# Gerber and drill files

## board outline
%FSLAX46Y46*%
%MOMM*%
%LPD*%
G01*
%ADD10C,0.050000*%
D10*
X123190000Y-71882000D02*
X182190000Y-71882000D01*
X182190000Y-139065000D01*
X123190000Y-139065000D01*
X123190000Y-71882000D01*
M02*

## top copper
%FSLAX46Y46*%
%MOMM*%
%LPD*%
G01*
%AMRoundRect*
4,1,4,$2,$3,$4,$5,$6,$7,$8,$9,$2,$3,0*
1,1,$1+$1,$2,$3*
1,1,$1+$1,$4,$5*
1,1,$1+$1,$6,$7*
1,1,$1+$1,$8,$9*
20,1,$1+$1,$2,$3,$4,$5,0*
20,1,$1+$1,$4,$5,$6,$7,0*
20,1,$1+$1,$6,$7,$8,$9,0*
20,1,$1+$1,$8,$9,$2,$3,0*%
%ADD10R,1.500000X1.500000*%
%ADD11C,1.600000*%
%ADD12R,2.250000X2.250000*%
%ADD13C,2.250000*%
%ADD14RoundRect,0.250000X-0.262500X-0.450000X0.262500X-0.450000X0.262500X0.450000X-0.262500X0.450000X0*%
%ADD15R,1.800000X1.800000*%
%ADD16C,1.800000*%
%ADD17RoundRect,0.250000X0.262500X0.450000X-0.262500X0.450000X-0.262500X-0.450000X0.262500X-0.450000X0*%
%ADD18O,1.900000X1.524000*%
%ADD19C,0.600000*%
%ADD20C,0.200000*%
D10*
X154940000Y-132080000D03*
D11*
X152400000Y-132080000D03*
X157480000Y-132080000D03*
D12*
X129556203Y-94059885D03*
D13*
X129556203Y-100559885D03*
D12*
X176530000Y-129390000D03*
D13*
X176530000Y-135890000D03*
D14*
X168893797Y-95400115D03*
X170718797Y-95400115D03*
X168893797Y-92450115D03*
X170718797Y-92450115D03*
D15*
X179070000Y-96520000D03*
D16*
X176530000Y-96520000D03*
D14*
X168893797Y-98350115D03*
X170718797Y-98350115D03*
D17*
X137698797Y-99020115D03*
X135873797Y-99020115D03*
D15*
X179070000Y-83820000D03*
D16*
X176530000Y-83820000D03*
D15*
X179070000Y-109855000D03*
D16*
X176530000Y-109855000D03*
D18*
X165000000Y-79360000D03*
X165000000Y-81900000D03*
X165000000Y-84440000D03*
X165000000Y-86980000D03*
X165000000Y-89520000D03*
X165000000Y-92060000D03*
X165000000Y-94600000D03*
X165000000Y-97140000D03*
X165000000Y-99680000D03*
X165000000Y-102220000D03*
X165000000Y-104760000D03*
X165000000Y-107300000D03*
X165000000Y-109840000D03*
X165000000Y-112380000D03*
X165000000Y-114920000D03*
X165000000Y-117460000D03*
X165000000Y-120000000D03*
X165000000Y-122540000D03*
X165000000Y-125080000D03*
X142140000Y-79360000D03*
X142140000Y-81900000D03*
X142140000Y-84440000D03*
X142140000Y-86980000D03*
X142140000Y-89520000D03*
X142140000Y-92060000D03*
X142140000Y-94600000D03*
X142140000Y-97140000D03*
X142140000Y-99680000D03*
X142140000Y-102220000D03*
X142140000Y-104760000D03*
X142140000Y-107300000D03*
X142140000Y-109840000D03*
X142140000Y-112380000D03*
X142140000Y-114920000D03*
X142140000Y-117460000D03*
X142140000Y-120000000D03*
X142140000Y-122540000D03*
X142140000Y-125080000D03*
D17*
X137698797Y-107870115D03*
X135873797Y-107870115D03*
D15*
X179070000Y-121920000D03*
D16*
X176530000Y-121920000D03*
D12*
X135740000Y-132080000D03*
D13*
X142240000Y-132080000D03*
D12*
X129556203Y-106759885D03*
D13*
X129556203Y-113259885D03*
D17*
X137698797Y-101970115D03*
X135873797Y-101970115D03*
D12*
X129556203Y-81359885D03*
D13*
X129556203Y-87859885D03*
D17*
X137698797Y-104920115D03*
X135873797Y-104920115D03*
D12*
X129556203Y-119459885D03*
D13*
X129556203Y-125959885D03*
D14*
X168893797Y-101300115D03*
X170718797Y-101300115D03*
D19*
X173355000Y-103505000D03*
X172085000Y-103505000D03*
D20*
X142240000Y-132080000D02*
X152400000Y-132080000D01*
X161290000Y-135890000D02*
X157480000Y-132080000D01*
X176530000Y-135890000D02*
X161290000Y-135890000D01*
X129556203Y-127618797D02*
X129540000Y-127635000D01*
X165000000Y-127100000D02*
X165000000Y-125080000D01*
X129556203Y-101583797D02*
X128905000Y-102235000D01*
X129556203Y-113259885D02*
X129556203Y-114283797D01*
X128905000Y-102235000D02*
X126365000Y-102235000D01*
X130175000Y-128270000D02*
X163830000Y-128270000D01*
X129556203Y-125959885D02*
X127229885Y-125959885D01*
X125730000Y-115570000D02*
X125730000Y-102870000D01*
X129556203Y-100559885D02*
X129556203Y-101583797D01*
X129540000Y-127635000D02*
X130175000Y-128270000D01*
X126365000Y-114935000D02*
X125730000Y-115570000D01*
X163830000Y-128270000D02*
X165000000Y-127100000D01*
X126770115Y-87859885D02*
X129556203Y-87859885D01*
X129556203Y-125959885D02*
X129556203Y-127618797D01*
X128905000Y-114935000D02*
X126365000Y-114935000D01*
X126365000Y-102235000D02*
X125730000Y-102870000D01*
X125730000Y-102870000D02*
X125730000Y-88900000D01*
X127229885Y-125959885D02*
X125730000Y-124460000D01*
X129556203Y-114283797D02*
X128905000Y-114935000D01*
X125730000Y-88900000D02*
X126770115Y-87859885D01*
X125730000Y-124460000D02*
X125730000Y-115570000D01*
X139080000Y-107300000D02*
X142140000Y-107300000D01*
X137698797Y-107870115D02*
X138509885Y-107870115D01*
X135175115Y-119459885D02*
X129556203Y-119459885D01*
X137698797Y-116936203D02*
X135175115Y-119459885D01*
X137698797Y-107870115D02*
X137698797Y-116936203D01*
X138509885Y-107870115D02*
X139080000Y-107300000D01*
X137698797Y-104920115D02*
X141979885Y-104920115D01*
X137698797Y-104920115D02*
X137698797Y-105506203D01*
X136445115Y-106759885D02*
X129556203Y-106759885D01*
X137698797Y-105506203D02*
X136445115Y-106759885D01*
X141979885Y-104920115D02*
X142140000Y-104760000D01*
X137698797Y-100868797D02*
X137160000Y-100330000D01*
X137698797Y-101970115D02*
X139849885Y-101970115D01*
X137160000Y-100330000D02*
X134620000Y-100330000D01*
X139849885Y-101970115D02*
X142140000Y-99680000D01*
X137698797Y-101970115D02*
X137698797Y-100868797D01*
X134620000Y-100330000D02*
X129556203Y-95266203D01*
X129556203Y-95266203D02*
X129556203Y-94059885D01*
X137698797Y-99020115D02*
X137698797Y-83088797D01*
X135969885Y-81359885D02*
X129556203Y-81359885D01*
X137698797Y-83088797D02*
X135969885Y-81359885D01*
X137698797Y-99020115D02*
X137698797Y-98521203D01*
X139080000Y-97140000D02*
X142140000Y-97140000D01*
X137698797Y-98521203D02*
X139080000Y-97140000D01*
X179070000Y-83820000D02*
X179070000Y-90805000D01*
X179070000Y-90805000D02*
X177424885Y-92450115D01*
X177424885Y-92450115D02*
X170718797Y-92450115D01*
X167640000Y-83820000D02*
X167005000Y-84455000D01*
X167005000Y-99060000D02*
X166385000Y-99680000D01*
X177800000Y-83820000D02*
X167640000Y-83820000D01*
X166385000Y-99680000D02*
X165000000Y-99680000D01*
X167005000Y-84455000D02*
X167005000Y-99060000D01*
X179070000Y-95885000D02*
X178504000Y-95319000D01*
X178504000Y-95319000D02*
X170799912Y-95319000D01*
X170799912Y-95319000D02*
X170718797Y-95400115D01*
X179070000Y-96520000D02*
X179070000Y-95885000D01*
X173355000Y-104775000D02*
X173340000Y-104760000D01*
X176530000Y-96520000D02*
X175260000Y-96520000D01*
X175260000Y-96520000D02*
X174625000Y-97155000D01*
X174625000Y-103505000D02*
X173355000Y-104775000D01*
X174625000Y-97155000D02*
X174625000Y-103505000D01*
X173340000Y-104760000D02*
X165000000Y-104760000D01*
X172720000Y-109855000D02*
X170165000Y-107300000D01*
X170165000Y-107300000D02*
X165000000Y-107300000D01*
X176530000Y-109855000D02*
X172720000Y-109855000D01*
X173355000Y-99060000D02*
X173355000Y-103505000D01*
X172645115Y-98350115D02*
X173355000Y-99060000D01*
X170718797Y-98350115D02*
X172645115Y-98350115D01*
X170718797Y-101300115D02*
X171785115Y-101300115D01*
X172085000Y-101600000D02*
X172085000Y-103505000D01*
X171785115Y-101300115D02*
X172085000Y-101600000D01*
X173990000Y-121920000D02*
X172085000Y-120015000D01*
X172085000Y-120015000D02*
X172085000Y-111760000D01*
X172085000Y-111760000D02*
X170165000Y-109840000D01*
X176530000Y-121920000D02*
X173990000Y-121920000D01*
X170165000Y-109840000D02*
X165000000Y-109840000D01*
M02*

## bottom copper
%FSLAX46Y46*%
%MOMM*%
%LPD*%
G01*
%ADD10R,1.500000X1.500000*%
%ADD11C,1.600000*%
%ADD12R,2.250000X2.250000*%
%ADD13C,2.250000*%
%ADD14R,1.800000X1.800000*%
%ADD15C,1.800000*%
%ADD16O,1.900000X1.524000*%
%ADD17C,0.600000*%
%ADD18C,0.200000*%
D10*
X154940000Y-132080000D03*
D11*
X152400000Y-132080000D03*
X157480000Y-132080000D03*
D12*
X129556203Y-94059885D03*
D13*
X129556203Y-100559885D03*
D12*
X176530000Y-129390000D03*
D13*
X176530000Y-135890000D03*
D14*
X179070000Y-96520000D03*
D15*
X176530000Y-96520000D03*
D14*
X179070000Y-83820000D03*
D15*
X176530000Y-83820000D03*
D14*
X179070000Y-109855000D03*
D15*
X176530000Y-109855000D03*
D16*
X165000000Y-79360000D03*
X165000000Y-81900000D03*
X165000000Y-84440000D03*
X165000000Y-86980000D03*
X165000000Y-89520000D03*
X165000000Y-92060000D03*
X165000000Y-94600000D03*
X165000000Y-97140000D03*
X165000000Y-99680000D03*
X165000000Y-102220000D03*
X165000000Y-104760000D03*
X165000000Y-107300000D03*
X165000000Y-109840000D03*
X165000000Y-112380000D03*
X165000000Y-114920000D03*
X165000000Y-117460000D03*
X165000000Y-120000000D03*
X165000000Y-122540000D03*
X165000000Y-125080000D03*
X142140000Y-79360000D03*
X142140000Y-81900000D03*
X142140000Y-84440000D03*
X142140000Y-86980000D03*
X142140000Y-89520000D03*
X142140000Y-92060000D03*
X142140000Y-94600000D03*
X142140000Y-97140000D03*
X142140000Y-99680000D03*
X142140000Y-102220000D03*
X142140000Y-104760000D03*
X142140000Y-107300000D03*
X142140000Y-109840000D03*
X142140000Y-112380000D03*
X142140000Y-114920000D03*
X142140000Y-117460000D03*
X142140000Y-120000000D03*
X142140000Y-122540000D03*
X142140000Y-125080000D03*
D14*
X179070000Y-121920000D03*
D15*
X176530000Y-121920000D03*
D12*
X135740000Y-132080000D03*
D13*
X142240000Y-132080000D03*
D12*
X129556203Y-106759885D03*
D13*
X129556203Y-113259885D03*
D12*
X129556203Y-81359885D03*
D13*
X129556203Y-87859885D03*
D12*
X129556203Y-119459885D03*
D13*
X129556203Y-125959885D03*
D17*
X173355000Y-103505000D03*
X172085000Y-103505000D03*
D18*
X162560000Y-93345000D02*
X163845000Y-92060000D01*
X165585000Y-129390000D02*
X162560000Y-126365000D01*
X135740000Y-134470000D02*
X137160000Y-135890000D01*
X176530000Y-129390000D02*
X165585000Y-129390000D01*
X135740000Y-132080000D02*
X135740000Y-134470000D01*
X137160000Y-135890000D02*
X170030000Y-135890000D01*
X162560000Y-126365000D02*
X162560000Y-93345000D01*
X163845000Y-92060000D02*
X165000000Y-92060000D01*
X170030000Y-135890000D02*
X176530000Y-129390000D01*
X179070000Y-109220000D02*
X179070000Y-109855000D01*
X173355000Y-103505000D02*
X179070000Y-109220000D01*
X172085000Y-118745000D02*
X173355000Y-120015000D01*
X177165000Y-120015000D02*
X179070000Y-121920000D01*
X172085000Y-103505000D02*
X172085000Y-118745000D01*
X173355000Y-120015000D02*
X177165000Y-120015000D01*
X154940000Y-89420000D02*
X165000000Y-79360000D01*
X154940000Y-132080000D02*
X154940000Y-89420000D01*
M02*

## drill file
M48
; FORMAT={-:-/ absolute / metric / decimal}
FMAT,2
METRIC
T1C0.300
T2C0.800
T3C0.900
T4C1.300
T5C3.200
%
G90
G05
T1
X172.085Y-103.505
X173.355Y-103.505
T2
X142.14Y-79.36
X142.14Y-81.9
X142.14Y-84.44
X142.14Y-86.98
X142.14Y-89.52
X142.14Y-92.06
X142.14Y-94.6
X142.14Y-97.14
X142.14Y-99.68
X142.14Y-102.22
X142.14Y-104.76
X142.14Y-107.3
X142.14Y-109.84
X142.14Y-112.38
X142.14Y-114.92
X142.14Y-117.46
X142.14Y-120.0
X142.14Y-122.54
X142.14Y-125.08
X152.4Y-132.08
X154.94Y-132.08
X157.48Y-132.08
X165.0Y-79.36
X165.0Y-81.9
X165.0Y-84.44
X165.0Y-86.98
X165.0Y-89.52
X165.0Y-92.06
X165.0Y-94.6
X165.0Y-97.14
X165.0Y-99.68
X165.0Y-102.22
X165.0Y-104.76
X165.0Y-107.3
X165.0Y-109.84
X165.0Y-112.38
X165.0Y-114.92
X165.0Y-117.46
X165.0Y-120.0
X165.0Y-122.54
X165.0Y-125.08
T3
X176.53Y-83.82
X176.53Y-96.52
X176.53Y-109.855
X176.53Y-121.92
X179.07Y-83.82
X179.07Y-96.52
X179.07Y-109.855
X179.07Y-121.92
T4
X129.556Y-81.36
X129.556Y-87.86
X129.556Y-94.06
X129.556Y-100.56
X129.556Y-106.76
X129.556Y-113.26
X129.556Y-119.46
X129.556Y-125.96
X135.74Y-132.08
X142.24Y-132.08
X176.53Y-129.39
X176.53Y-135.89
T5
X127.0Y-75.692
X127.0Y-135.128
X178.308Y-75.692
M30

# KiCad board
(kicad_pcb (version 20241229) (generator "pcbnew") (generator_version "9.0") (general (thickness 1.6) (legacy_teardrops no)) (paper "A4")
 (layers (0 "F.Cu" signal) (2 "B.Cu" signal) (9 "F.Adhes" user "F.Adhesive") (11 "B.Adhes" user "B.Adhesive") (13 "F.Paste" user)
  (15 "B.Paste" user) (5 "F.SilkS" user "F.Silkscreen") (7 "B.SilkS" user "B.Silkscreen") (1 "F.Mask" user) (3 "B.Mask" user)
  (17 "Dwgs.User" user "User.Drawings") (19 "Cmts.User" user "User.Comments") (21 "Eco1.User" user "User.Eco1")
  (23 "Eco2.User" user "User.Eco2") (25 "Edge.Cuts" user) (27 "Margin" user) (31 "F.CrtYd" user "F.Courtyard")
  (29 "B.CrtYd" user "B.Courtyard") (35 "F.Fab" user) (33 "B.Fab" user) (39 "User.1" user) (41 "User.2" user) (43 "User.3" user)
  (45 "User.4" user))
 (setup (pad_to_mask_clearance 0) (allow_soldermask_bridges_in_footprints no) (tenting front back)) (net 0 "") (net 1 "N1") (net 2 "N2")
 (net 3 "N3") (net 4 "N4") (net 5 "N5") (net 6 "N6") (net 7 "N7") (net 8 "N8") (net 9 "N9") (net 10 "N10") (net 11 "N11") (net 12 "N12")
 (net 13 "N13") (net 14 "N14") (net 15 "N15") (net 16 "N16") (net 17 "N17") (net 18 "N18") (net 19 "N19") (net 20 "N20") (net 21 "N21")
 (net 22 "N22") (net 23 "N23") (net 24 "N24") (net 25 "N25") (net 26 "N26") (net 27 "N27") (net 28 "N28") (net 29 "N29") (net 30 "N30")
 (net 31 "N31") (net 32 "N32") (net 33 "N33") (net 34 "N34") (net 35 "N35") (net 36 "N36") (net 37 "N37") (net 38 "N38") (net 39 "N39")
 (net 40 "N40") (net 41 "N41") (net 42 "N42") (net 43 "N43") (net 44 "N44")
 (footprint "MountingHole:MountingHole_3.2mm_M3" (layer "F.Cu") (at 178.308 75.692)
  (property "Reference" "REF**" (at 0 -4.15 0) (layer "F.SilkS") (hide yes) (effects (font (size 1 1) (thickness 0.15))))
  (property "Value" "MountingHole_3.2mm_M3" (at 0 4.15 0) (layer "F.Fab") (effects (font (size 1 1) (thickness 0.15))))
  (pad "" np_thru_hole circle (at 0 0) (size 3.2 3.2) (drill 3.2) (layers "*.Cu" "*.Mask")))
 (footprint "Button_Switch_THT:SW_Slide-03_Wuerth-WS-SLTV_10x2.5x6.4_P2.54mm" (layer "F.Cu") (at 154.94 132.08)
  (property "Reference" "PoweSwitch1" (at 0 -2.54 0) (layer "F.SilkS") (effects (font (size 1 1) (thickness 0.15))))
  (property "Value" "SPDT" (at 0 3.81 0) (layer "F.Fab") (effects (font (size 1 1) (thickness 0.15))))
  (pad "1" thru_hole rect (at 0 0) (size 1.5 1.5) (drill 0.8) (layers "*.Cu" "*.Mask") (remove_unused_layers no) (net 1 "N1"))
  (pad "2" thru_hole circle (at -2.54 0) (size 1.6 1.6) (drill 0.8) (layers "*.Cu" "*.Mask") (remove_unused_layers no) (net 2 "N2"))
  (pad "3" thru_hole circle (at 2.54 0) (size 1.6 1.6) (drill 0.8) (layers "*.Cu" "*.Mask") (remove_unused_layers no) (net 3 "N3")))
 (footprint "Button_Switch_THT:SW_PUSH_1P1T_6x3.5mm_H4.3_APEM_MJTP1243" (layer "F.Cu") (at 129.556203 94.059885 -90)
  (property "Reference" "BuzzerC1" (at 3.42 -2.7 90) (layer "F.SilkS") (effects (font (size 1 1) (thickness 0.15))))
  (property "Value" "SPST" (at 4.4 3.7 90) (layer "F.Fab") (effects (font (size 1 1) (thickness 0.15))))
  (pad "1" thru_hole rect (at 0 0) (size 2.25 2.25) (drill 1.3) (layers "*.Cu" "*.Mask") (remove_unused_layers no) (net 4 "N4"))
  (pad "2" thru_hole circle (at 6.5 0) (size 2.25 2.25) (drill 1.3) (layers "*.Cu" "*.Mask") (remove_unused_layers no) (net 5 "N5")))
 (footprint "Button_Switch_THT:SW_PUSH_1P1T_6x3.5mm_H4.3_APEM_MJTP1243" (layer "F.Cu") (at 176.53 129.39 -90)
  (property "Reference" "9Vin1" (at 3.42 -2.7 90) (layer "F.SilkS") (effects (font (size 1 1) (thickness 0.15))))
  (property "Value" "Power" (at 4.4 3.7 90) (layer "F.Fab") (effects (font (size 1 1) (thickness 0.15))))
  (pad "1" thru_hole rect (at 0 0) (size 2.25 2.25) (drill 1.3) (layers "*.Cu" "*.Mask") (remove_unused_layers no) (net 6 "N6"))
  (pad "2" thru_hole circle (at 6.5 0) (size 2.25 2.25) (drill 1.3) (layers "*.Cu" "*.Mask") (remove_unused_layers no) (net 3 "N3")))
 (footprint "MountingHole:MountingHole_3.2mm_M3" (layer "F.Cu") (at 127 135.128)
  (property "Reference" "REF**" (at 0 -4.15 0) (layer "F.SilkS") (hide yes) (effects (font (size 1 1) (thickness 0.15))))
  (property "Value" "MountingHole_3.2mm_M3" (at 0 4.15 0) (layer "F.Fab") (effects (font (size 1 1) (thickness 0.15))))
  (pad "" np_thru_hole circle (at 0 0) (size 3.2 3.2) (drill 3.2) (layers "*.Cu" "*.Mask")))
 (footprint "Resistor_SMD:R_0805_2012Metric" (layer "F.Cu") (at 169.806297 95.400115)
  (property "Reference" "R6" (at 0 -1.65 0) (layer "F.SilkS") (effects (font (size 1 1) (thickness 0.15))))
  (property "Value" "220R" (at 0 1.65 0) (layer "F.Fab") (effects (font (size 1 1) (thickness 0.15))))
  (pad "1" smd roundrect (at -0.9125 0) (size 1.025 1.4) (layers "F.Cu" "F.Mask" "F.Paste") (roundrect_rratio 0.243902) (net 6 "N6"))
  (pad "2" smd roundrect (at 0.9125 0) (size 1.025 1.4) (layers "F.Cu" "F.Mask" "F.Paste") (roundrect_rratio 0.243902) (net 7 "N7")))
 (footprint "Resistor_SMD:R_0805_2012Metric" (layer "F.Cu") (at 169.806297 92.450115)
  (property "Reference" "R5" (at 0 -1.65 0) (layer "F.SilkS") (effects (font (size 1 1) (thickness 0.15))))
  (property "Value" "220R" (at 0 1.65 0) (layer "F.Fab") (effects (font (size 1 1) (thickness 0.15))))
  (pad "1" smd roundrect (at -0.9125 0) (size 1.025 1.4) (layers "F.Cu" "F.Mask" "F.Paste") (roundrect_rratio 0.243902) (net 6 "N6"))
  (pad "2" smd roundrect (at 0.9125 0) (size 1.025 1.4) (layers "F.Cu" "F.Mask" "F.Paste") (roundrect_rratio 0.243902) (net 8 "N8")))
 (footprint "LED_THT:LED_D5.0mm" (layer "F.Cu") (at 179.07 96.52 180)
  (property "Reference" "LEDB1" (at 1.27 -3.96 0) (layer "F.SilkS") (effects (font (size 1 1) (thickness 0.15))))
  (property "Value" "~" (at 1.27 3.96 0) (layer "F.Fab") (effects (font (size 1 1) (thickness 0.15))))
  (pad "1" thru_hole rect (at 0 0 180) (size 1.8 1.8) (drill 0.9) (layers "*.Cu" "*.Mask") (remove_unused_layers no) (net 7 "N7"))
  (pad "2" thru_hole circle (at 2.54 0 180) (size 1.8 1.8) (drill 0.9) (layers "*.Cu" "*.Mask") (remove_unused_layers no) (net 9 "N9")))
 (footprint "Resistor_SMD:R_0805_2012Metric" (layer "F.Cu") (at 169.806297 98.350115)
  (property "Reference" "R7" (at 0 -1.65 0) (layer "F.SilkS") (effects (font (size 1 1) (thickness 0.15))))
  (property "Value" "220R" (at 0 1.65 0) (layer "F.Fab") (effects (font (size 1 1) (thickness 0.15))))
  (pad "1" smd roundrect (at -0.9125 0) (size 1.025 1.4) (layers "F.Cu" "F.Mask" "F.Paste") (roundrect_rratio 0.243902) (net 6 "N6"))
  (pad "2" smd roundrect (at 0.9125 0) (size 1.025 1.4) (layers "F.Cu" "F.Mask" "F.Paste") (roundrect_rratio 0.243902) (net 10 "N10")))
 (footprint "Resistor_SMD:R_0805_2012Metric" (layer "F.Cu") (at 136.786297 99.020115 180)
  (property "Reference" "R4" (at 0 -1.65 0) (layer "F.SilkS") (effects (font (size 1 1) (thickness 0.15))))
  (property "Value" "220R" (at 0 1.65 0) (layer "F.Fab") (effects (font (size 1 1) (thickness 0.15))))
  (pad "1" smd roundrect (at -0.9125 0 180) (size 1.025 1.4) (layers "F.Cu" "F.Mask" "F.Paste") (roundrect_rratio 0.243902) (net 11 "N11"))
  (pad "2" smd roundrect (at 0.9125 0 180) (size 1.025 1.4) (layers "F.Cu" "F.Mask" "F.Paste") (roundrect_rratio 0.243902) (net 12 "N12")))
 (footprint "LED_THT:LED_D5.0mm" (layer "F.Cu") (at 179.07 83.82 180)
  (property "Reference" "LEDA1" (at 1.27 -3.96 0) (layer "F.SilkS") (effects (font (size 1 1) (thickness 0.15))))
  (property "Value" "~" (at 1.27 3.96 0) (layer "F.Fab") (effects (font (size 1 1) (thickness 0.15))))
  (pad "1" thru_hole rect (at 0 0 180) (size 1.8 1.8) (drill 0.9) (layers "*.Cu" "*.Mask") (remove_unused_layers no) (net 8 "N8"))
  (pad "2" thru_hole circle (at 2.54 0 180) (size 1.8 1.8) (drill 0.9) (layers "*.Cu" "*.Mask") (remove_unused_layers no) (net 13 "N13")))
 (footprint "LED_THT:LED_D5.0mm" (layer "F.Cu") (at 179.07 109.855 180)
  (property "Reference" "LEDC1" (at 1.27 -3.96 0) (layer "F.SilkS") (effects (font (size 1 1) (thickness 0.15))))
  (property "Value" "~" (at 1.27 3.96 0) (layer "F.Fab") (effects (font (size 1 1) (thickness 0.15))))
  (pad "1" thru_hole rect (at 0 0 180) (size 1.8 1.8) (drill 0.9) (layers "*.Cu" "*.Mask") (remove_unused_layers no) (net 10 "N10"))
  (pad "2" thru_hole circle (at 2.54 0 180) (size 1.8 1.8) (drill 0.9) (layers "*.Cu" "*.Mask") (remove_unused_layers no) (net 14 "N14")))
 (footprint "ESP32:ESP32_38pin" (layer "F.Cu") (at 153.456183 102.385111 180)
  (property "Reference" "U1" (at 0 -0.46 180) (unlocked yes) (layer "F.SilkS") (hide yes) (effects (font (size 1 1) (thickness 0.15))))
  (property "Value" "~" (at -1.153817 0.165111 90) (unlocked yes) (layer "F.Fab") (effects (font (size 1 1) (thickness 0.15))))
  (pad "1" thru_hole oval (at -11.543817 23.025111 90) (size 1.524 1.9) (drill 0.8) (layers "*.Cu" "*.Mask") (remove_unused_layers no)
   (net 1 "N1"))
  (pad "2" thru_hole oval (at -11.543817 20.485111 90) (size 1.524 1.9) (drill 0.8) (layers "*.Cu" "*.Mask") (remove_unused_layers no)
   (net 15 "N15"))
  (pad "3" thru_hole oval (at -11.543817 17.945111 90) (size 1.524 1.9) (drill 0.8) (layers "*.Cu" "*.Mask") (remove_unused_layers no)
   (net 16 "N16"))
  (pad "4" thru_hole oval (at -11.543817 15.405111 90) (size 1.524 1.9) (drill 0.8) (layers "*.Cu" "*.Mask") (remove_unused_layers no)
   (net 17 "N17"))
  (pad "5" thru_hole oval (at -11.543817 12.865111 90) (size 1.524 1.9) (drill 0.8) (layers "*.Cu" "*.Mask") (remove_unused_layers no)
   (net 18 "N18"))
  (pad "6" thru_hole oval (at -11.543817 10.325111 90) (size 1.524 1.9) (drill 0.8) (layers "*.Cu" "*.Mask") (remove_unused_layers no)
   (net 6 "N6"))
  (pad "7" thru_hole oval (at -11.543817 7.785111 90) (size 1.524 1.9) (drill 0.8) (layers "*.Cu" "*.Mask") (remove_unused_layers no)
   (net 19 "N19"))
  (pad "8" thru_hole oval (at -11.543817 5.245111 90) (size 1.524 1.9) (drill 0.8) (layers "*.Cu" "*.Mask") (remove_unused_layers no)
   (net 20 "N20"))
  (pad "9" thru_hole oval (at -11.543817 2.705111 90) (size 1.524 1.9) (drill 0.8) (layers "*.Cu" "*.Mask") (remove_unused_layers no)
   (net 13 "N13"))
  (pad "10" thru_hole oval (at -11.543817 0.165111 90) (size 1.524 1.9) (drill 0.8) (layers "*.Cu" "*.Mask") (remove_unused_layers no)
   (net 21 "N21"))
  (pad "11" thru_hole oval (at -11.543817 -2.374889 90) (size 1.524 1.9) (drill 0.8) (layers "*.Cu" "*.Mask") (remove_unused_layers no)
   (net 9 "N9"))
  (pad "12" thru_hole oval (at -11.543817 -4.914889 90) (size 1.524 1.9) (drill 0.8) (layers "*.Cu" "*.Mask") (remove_unused_layers no)
   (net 14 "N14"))
  (pad "13" thru_hole oval (at -11.543817 -7.454889 90) (size 1.524 1.9) (drill 0.8) (layers "*.Cu" "*.Mask") (remove_unused_layers no)
   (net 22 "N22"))
  (pad "14" thru_hole oval (at -11.543817 -9.994889 90) (size 1.524 1.9) (drill 0.8) (layers "*.Cu" "*.Mask") (remove_unused_layers no)
   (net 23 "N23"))
  (pad "15" thru_hole oval (at -11.543817 -12.534889 90) (size 1.524 1.9) (drill 0.8) (layers "*.Cu" "*.Mask") (remove_unused_layers no)
   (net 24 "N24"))
  (pad "16" thru_hole oval (at -11.543817 -15.074889 90) (size 1.524 1.9) (drill 0.8) (layers "*.Cu" "*.Mask") (remove_unused_layers no)
   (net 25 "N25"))
  (pad "17" thru_hole oval (at -11.543817 -17.614889 90) (size 1.524 1.9) (drill 0.8) (layers "*.Cu" "*.Mask") (remove_unused_layers no)
   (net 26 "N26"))
  (pad "18" thru_hole oval (at -11.543817 -20.154889 90) (size 1.524 1.9) (drill 0.8) (layers "*.Cu" "*.Mask") (remove_unused_layers no)
   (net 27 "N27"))
  (pad "19" thru_hole oval (at -11.543817 -22.694889 90) (size 1.524 1.9) (drill 0.8) (layers "*.Cu" "*.Mask") (remove_unused_layers no)
   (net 5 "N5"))
  (pad "20" thru_hole oval (at 11.316183 23.025111 90) (size 1.524 1.9) (drill 0.8) (layers "*.Cu" "*.Mask") (remove_unused_layers no)
   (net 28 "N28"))
  (pad "21" thru_hole oval (at 11.316183 20.485111 90) (size 1.524 1.9) (drill 0.8) (layers "*.Cu" "*.Mask") (remove_unused_layers no)
   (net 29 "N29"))
  (pad "22" thru_hole oval (at 11.316183 17.945111 90) (size 1.524 1.9) (drill 0.8) (layers "*.Cu" "*.Mask") (remove_unused_layers no)
   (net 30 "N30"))
  (pad "23" thru_hole oval (at 11.316183 15.405111 90) (size 1.524 1.9) (drill 0.8) (layers "*.Cu" "*.Mask") (remove_unused_layers no)
   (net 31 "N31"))
  (pad "24" thru_hole oval (at 11.316183 12.865111 90) (size 1.524 1.9) (drill 0.8) (layers "*.Cu" "*.Mask") (remove_unused_layers no)
   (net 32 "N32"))
  (pad "25" thru_hole oval (at 11.316183 10.325111 90) (size 1.524 1.9) (drill 0.8) (layers "*.Cu" "*.Mask") (remove_unused_layers no)
   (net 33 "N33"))
  (pad "26" thru_hole oval (at 11.316183 7.785111 90) (size 1.524 1.9) (drill 0.8) (layers "*.Cu" "*.Mask") (remove_unused_layers no)
   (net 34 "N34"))
  (pad "27" thru_hole oval (at 11.316183 5.245111 90) (size 1.524 1.9) (drill 0.8) (layers "*.Cu" "*.Mask") (remove_unused_layers no)
   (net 11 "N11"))
  (pad "28" thru_hole oval (at 11.316183 2.705111 90) (size 1.524 1.9) (drill 0.8) (layers "*.Cu" "*.Mask") (remove_unused_layers no)
   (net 4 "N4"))
  (pad "29" thru_hole oval (at 11.316183 0.165111 90) (size 1.524 1.9) (drill 0.8) (layers "*.Cu" "*.Mask") (remove_unused_layers no)
   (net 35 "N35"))
  (pad "30" thru_hole oval (at 11.316183 -2.374889 90) (size 1.524 1.9) (drill 0.8) (layers "*.Cu" "*.Mask") (remove_unused_layers no)
   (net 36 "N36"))
  (pad "31" thru_hole oval (at 11.316183 -4.914889 90) (size 1.524 1.9) (drill 0.8) (layers "*.Cu" "*.Mask") (remove_unused_layers no)
   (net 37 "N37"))
  (pad "32" thru_hole oval (at 11.316183 -7.454889 90) (size 1.524 1.9) (drill 0.8) (layers "*.Cu" "*.Mask") (remove_unused_layers no)
   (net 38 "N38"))
  (pad "33" thru_hole oval (at 11.316183 -9.994889 90) (size 1.524 1.9) (drill 0.8) (layers "*.Cu" "*.Mask") (remove_unused_layers no)
   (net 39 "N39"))
  (pad "34" thru_hole oval (at 11.316183 -12.534889 90) (size 1.524 1.9) (drill 0.8) (layers "*.Cu" "*.Mask") (remove_unused_layers no)
   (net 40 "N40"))
  (pad "35" thru_hole oval (at 11.316183 -15.074889 90) (size 1.524 1.9) (drill 0.8) (layers "*.Cu" "*.Mask") (remove_unused_layers no)
   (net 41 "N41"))
  (pad "36" thru_hole oval (at 11.316183 -17.614889 90) (size 1.524 1.9) (drill 0.8) (layers "*.Cu" "*.Mask") (remove_unused_layers no)
   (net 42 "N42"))
  (pad "37" thru_hole oval (at 11.316183 -20.154889 90) (size 1.524 1.9) (drill 0.8) (layers "*.Cu" "*.Mask") (remove_unused_layers no)
   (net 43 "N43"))
  (pad "38" thru_hole oval (at 11.316183 -22.694889 90) (size 1.524 1.9) (drill 0.8) (layers "*.Cu" "*.Mask") (remove_unused_layers no)
   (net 12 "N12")))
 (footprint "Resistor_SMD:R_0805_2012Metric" (layer "F.Cu") (at 136.786297 107.870115 180)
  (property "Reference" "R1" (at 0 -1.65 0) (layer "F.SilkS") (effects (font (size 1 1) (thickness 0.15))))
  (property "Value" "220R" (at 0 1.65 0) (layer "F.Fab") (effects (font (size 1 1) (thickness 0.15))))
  (pad "1" smd roundrect (at -0.9125 0 180) (size 1.025 1.4) (layers "F.Cu" "F.Mask" "F.Paste") (roundrect_rratio 0.243902) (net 37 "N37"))
  (pad "2" smd roundrect (at 0.9125 0 180) (size 1.025 1.4) (layers "F.Cu" "F.Mask" "F.Paste") (roundrect_rratio 0.243902) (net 12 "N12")))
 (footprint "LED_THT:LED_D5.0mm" (layer "F.Cu") (at 179.07 121.92 180)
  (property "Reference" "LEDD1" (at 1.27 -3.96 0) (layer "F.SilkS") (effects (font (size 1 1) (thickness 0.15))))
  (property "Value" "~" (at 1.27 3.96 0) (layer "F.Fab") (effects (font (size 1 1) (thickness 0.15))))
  (pad "1" thru_hole rect (at 0 0 180) (size 1.8 1.8) (drill 0.9) (layers "*.Cu" "*.Mask") (remove_unused_layers no) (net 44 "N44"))
  (pad "2" thru_hole circle (at 2.54 0 180) (size 1.8 1.8) (drill 0.9) (layers "*.Cu" "*.Mask") (remove_unused_layers no) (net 22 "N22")))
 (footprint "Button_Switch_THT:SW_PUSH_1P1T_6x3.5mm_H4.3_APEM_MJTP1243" (layer "F.Cu") (at 135.74 132.08)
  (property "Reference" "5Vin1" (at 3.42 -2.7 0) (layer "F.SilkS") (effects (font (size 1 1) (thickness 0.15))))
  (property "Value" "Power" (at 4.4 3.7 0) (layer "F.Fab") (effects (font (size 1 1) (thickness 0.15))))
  (pad "1" thru_hole rect (at 0 0 90) (size 2.25 2.25) (drill 1.3) (layers "*.Cu" "*.Mask") (remove_unused_layers no) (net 6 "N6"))
  (pad "2" thru_hole circle (at 6.5 0 90) (size 2.25 2.25) (drill 1.3) (layers "*.Cu" "*.Mask") (remove_unused_layers no) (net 2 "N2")))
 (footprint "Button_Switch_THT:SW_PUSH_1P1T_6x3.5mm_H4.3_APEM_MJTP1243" (layer "F.Cu") (at 129.556203 106.759885 -90)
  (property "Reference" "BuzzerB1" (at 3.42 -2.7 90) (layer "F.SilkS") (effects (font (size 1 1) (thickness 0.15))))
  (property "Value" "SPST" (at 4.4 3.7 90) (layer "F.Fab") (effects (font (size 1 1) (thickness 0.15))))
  (pad "1" thru_hole rect (at 0 0) (size 2.25 2.25) (drill 1.3) (layers "*.Cu" "*.Mask") (remove_unused_layers no) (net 36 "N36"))
  (pad "2" thru_hole circle (at 6.5 0) (size 2.25 2.25) (drill 1.3) (layers "*.Cu" "*.Mask") (remove_unused_layers no) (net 5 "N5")))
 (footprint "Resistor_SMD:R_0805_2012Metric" (layer "F.Cu") (at 136.786297 101.970115 180)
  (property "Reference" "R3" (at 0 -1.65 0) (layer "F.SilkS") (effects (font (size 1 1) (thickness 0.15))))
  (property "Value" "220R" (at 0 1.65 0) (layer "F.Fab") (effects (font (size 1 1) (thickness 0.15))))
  (pad "1" smd roundrect (at -0.9125 0 180) (size 1.025 1.4) (layers "F.Cu" "F.Mask" "F.Paste") (roundrect_rratio 0.243902) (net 4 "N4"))
  (pad "2" smd roundrect (at 0.9125 0 180) (size 1.025 1.4) (layers "F.Cu" "F.Mask" "F.Paste") (roundrect_rratio 0.243902) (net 12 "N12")))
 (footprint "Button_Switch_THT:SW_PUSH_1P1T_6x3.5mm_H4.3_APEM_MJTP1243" (layer "F.Cu") (at 129.556203 81.359885 -90)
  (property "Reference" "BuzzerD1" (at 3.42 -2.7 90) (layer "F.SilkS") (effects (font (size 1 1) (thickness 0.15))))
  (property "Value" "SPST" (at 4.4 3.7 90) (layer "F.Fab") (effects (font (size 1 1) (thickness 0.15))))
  (pad "1" thru_hole rect (at 0 0) (size 2.25 2.25) (drill 1.3) (layers "*.Cu" "*.Mask") (remove_unused_layers no) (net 11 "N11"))
  (pad "2" thru_hole circle (at 6.5 0) (size 2.25 2.25) (drill 1.3) (layers "*.Cu" "*.Mask") (remove_unused_layers no) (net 5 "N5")))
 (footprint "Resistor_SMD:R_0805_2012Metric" (layer "F.Cu") (at 136.786297 104.920115 180)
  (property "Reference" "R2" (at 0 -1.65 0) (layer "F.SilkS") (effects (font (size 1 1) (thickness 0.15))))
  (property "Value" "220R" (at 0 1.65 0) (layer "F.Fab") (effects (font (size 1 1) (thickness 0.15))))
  (pad "1" smd roundrect (at -0.9125 0 180) (size 1.025 1.4) (layers "F.Cu" "F.Mask" "F.Paste") (roundrect_rratio 0.243902) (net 36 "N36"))
  (pad "2" smd roundrect (at 0.9125 0 180) (size 1.025 1.4) (layers "F.Cu" "F.Mask" "F.Paste") (roundrect_rratio 0.243902) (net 12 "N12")))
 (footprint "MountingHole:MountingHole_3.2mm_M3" (layer "F.Cu") (at 127 75.692)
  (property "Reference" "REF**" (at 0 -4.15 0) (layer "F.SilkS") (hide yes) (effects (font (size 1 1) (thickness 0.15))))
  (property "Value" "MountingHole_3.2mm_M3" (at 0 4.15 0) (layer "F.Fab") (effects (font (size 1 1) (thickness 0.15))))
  (pad "" np_thru_hole circle (at 0 0) (size 3.2 3.2) (drill 3.2) (layers "*.Cu" "*.Mask")))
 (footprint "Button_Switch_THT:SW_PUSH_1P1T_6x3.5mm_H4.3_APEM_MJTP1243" (layer "F.Cu") (at 129.556203 119.459885 -90)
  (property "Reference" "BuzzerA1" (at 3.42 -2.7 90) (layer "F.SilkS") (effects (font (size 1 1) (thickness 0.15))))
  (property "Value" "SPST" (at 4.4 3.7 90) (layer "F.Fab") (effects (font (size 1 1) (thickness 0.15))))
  (pad "1" thru_hole rect (at 0 0) (size 2.25 2.25) (drill 1.3) (layers "*.Cu" "*.Mask") (remove_unused_layers no) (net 37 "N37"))
  (pad "2" thru_hole circle (at 6.5 0) (size 2.25 2.25) (drill 1.3) (layers "*.Cu" "*.Mask") (remove_unused_layers no) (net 5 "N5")))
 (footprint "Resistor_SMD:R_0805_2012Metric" (layer "F.Cu") (at 169.806297 101.300115)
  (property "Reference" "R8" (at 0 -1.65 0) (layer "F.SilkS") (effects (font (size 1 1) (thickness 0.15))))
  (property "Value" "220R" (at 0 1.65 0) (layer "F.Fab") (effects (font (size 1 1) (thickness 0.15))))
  (pad "1" smd roundrect (at -0.9125 0) (size 1.025 1.4) (layers "F.Cu" "F.Mask" "F.Paste") (roundrect_rratio 0.243902) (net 6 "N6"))
  (pad "2" smd roundrect (at 0.9125 0) (size 1.025 1.4) (layers "F.Cu" "F.Mask" "F.Paste") (roundrect_rratio 0.243902) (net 44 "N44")))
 (gr_rect (start 123.19 71.882) (end 182.19 139.065) (stroke (width 0.05) (type solid)) (fill no) (layer "Edge.Cuts"))
 (segment (start 162.56 93.345) (end 163.845 92.06) (width 0.2) (layer "B.Cu") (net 6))
 (segment (start 165.585 129.39) (end 162.56 126.365) (width 0.2) (layer "B.Cu") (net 6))
 (segment (start 135.74 134.47) (end 137.16 135.89) (width 0.2) (layer "B.Cu") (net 6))
 (segment (start 176.53 129.39) (end 165.585 129.39) (width 0.2) (layer "B.Cu") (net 6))
 (segment (start 135.74 132.08) (end 135.74 134.47) (width 0.2) (layer "B.Cu") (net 6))
 (segment (start 137.16 135.89) (end 170.03 135.89) (width 0.2) (layer "B.Cu") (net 6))
 (segment (start 162.56 126.365) (end 162.56 93.345) (width 0.2) (layer "B.Cu") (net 6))
 (segment (start 163.845 92.06) (end 165 92.06) (width 0.2) (layer "B.Cu") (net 6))
 (segment (start 170.03 135.89) (end 176.53 129.39) (width 0.2) (layer "B.Cu") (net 6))
 (segment (start 142.24 132.08) (end 152.4 132.08) (width 0.2) (layer "F.Cu") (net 2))
 (segment (start 161.29 135.89) (end 157.48 132.08) (width 0.2) (layer "F.Cu") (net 3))
 (segment (start 176.53 135.89) (end 161.29 135.89) (width 0.2) (layer "F.Cu") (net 3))
 (segment (start 129.556203 127.618797) (end 129.54 127.635) (width 0.2) (layer "F.Cu") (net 5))
 (segment (start 165 127.1) (end 165 125.08) (width 0.2) (layer "F.Cu") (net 5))
 (segment (start 129.556203 101.583797) (end 128.905 102.235) (width 0.2) (layer "F.Cu") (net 5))
 (segment (start 129.556203 113.259885) (end 129.556203 114.283797) (width 0.2) (layer "F.Cu") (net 5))
 (segment (start 128.905 102.235) (end 126.365 102.235) (width 0.2) (layer "F.Cu") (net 5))
 (segment (start 130.175 128.27) (end 163.83 128.27) (width 0.2) (layer "F.Cu") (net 5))
 (segment (start 129.556203 125.959885) (end 127.229885 125.959885) (width 0.2) (layer "F.Cu") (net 5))
 (segment (start 125.73 115.57) (end 125.73 102.87) (width 0.2) (layer "F.Cu") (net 5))
 (segment (start 129.556203 100.559885) (end 129.556203 101.583797) (width 0.2) (layer "F.Cu") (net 5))
 (segment (start 129.54 127.635) (end 130.175 128.27) (width 0.2) (layer "F.Cu") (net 5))
 (segment (start 126.365 114.935) (end 125.73 115.57) (width 0.2) (layer "F.Cu") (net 5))
 (segment (start 163.83 128.27) (end 165 127.1) (width 0.2) (layer "F.Cu") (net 5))
 (segment (start 126.770115 87.859885) (end 129.556203 87.859885) (width 0.2) (layer "F.Cu") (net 5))
 (segment (start 129.556203 125.959885) (end 129.556203 127.618797) (width 0.2) (layer "F.Cu") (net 5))
 (segment (start 128.905 114.935) (end 126.365 114.935) (width 0.2) (layer "F.Cu") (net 5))
 (segment (start 126.365 102.235) (end 125.73 102.87) (width 0.2) (layer "F.Cu") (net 5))
 (segment (start 125.73 102.87) (end 125.73 88.9) (width 0.2) (layer "F.Cu") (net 5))
 (segment (start 127.229885 125.959885) (end 125.73 124.46) (width 0.2) (layer "F.Cu") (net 5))
 (segment (start 129.556203 114.283797) (end 128.905 114.935) (width 0.2) (layer "F.Cu") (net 5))
 (segment (start 125.73 88.9) (end 126.770115 87.859885) (width 0.2) (layer "F.Cu") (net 5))
 (segment (start 125.73 124.46) (end 125.73 115.57) (width 0.2) (layer "F.Cu") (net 5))
 (segment (start 139.08 107.3) (end 142.14 107.3) (width 0.2) (layer "F.Cu") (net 37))
 (segment (start 137.698797 107.870115) (end 138.509885 107.870115) (width 0.2) (layer "F.Cu") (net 37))
 (segment (start 135.175115 119.459885) (end 129.556203 119.459885) (width 0.2) (layer "F.Cu") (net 37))
 (segment (start 137.698797 116.936203) (end 135.175115 119.459885) (width 0.2) (layer "F.Cu") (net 37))
 (segment (start 137.698797 107.870115) (end 137.698797 116.936203) (width 0.2) (layer "F.Cu") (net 37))
 (segment (start 138.509885 107.870115) (end 139.08 107.3) (width 0.2) (layer "F.Cu") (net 37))
 (segment (start 137.698797 104.920115) (end 141.979885 104.920115) (width 0.2) (layer "F.Cu") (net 36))
 (segment (start 137.698797 104.920115) (end 137.698797 105.506203) (width 0.2) (layer "F.Cu") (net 36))
 (segment (start 136.445115 106.759885) (end 129.556203 106.759885) (width 0.2) (layer "F.Cu") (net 36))
 (segment (start 137.698797 105.506203) (end 136.445115 106.759885) (width 0.2) (layer "F.Cu") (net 36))
 (segment (start 141.979885 104.920115) (end 142.14 104.76) (width 0.2) (layer "F.Cu") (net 36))
 (segment (start 137.698797 100.868797) (end 137.16 100.33) (width 0.2) (layer "F.Cu") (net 4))
 (segment (start 137.698797 101.970115) (end 139.849885 101.970115) (width 0.2) (layer "F.Cu") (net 4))
 (segment (start 137.16 100.33) (end 134.62 100.33) (width 0.2) (layer "F.Cu") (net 4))
 (segment (start 139.849885 101.970115) (end 142.14 99.68) (width 0.2) (layer "F.Cu") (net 4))
 (segment (start 137.698797 101.970115) (end 137.698797 100.868797) (width 0.2) (layer "F.Cu") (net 4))
 (segment (start 134.62 100.33) (end 129.556203 95.266203) (width 0.2) (layer "F.Cu") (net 4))
 (segment (start 129.556203 95.266203) (end 129.556203 94.059885) (width 0.2) (layer "F.Cu") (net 4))
 (segment (start 137.698797 99.020115) (end 137.698797 83.088797) (width 0.2) (layer "F.Cu") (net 11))
 (segment (start 135.969885 81.359885) (end 129.556203 81.359885) (width 0.2) (layer "F.Cu") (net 11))
 (segment (start 137.698797 83.088797) (end 135.969885 81.359885) (width 0.2) (layer "F.Cu") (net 11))
 (segment (start 137.698797 99.020115) (end 137.698797 98.521203) (width 0.2) (layer "F.Cu") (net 11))
 (segment (start 139.08 97.14) (end 142.14 97.14) (width 0.2) (layer "F.Cu") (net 11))
 (segment (start 137.698797 98.521203) (end 139.08 97.14) (width 0.2) (layer "F.Cu") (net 11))
 (segment (start 179.07 83.82) (end 179.07 90.805) (width 0.2) (layer "F.Cu") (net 8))
 (segment (start 179.07 90.805) (end 177.424885 92.450115) (width 0.2) (layer "F.Cu") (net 8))
 (segment (start 177.424885 92.450115) (end 170.718797 92.450115) (width 0.2) (layer "F.Cu") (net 8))
 (segment (start 167.64 83.82) (end 167.005 84.455) (width 0.2) (layer "F.Cu") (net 13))
 (segment (start 167.005 99.06) (end 166.385 99.68) (width 0.2) (layer "F.Cu") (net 13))
 (segment (start 177.8 83.82) (end 167.64 83.82) (width 0.2) (layer "F.Cu") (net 13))
 (segment (start 166.385 99.68) (end 165 99.68) (width 0.2) (layer "F.Cu") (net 13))
 (segment (start 167.005 84.455) (end 167.005 99.06) (width 0.2) (layer "F.Cu") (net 13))
 (segment (start 179.07 95.885) (end 178.504 95.319) (width 0.2) (layer "F.Cu") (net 7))
 (segment (start 178.504 95.319) (end 170.799912 95.319) (width 0.2) (layer "F.Cu") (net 7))
 (segment (start 170.799912 95.319) (end 170.718797 95.400115) (width 0.2) (layer "F.Cu") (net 7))
 (segment (start 179.07 96.52) (end 179.07 95.885) (width 0.2) (layer "F.Cu") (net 7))
 (segment (start 173.355 104.775) (end 173.34 104.76) (width 0.2) (layer "F.Cu") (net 9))
 (segment (start 176.53 96.52) (end 175.26 96.52) (width 0.2) (layer "F.Cu") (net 9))
 (segment (start 175.26 96.52) (end 174.625 97.155) (width 0.2) (layer "F.Cu") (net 9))
 (segment (start 174.625 103.505) (end 173.355 104.775) (width 0.2) (layer "F.Cu") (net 9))
 (segment (start 174.625 97.155) (end 174.625 103.505) (width 0.2) (layer "F.Cu") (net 9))
 (segment (start 173.34 104.76) (end 165 104.76) (width 0.2) (layer "F.Cu") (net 9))
 (segment (start 172.72 109.855) (end 170.165 107.3) (width 0.2) (layer "F.Cu") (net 14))
 (segment (start 170.165 107.3) (end 165 107.3) (width 0.2) (layer "F.Cu") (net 14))
 (segment (start 176.53 109.855) (end 172.72 109.855) (width 0.2) (layer "F.Cu") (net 14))
 (segment (start 173.355 99.06) (end 173.355 103.505) (width 0.2) (layer "F.Cu") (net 10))
 (segment (start 172.645115 98.350115) (end 173.355 99.06) (width 0.2) (layer "F.Cu") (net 10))
 (segment (start 170.718797 98.350115) (end 172.645115 98.350115) (width 0.2) (layer "F.Cu") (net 10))
 (via (at 173.355 103.505) (size 0.6) (drill 0.3) (layers "F.Cu" "B.Cu") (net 10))
 (segment (start 179.07 109.22) (end 179.07 109.855) (width 0.2) (layer "B.Cu") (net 10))
 (segment (start 173.355 103.505) (end 179.07 109.22) (width 0.2) (layer "B.Cu") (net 10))
 (segment (start 170.718797 101.300115) (end 171.785115 101.300115) (width 0.2) (layer "F.Cu") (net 44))
 (segment (start 172.085 101.6) (end 172.085 103.505) (width 0.2) (layer "F.Cu") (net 44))
 (segment (start 171.785115 101.300115) (end 172.085 101.6) (width 0.2) (layer "F.Cu") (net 44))
 (via (at 172.085 103.505) (size 0.6) (drill 0.3) (layers "F.Cu" "B.Cu") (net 44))
 (segment (start 172.085 118.745) (end 173.355 120.015) (width 0.2) (layer "B.Cu") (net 44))
 (segment (start 177.165 120.015) (end 179.07 121.92) (width 0.2) (layer "B.Cu") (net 44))
 (segment (start 172.085 103.505) (end 172.085 118.745) (width 0.2) (layer "B.Cu") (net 44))
 (segment (start 173.355 120.015) (end 177.165 120.015) (width 0.2) (layer "B.Cu") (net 44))
 (segment (start 173.99 121.92) (end 172.085 120.015) (width 0.2) (layer "F.Cu") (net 22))
 (segment (start 172.085 120.015) (end 172.085 111.76) (width 0.2) (layer "F.Cu") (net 22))
 (segment (start 172.085 111.76) (end 170.165 109.84) (width 0.2) (layer "F.Cu") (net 22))
 (segment (start 176.53 121.92) (end 173.99 121.92) (width 0.2) (layer "F.Cu") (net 22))
 (segment (start 170.165 109.84) (end 165 109.84) (width 0.2) (layer "F.Cu") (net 22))
 (segment (start 154.94 89.42) (end 165 79.36) (width 0.2) (layer "B.Cu") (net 1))
 (segment (start 154.94 132.08) (end 154.94 89.42) (width 0.2) (layer "B.Cu") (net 1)))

